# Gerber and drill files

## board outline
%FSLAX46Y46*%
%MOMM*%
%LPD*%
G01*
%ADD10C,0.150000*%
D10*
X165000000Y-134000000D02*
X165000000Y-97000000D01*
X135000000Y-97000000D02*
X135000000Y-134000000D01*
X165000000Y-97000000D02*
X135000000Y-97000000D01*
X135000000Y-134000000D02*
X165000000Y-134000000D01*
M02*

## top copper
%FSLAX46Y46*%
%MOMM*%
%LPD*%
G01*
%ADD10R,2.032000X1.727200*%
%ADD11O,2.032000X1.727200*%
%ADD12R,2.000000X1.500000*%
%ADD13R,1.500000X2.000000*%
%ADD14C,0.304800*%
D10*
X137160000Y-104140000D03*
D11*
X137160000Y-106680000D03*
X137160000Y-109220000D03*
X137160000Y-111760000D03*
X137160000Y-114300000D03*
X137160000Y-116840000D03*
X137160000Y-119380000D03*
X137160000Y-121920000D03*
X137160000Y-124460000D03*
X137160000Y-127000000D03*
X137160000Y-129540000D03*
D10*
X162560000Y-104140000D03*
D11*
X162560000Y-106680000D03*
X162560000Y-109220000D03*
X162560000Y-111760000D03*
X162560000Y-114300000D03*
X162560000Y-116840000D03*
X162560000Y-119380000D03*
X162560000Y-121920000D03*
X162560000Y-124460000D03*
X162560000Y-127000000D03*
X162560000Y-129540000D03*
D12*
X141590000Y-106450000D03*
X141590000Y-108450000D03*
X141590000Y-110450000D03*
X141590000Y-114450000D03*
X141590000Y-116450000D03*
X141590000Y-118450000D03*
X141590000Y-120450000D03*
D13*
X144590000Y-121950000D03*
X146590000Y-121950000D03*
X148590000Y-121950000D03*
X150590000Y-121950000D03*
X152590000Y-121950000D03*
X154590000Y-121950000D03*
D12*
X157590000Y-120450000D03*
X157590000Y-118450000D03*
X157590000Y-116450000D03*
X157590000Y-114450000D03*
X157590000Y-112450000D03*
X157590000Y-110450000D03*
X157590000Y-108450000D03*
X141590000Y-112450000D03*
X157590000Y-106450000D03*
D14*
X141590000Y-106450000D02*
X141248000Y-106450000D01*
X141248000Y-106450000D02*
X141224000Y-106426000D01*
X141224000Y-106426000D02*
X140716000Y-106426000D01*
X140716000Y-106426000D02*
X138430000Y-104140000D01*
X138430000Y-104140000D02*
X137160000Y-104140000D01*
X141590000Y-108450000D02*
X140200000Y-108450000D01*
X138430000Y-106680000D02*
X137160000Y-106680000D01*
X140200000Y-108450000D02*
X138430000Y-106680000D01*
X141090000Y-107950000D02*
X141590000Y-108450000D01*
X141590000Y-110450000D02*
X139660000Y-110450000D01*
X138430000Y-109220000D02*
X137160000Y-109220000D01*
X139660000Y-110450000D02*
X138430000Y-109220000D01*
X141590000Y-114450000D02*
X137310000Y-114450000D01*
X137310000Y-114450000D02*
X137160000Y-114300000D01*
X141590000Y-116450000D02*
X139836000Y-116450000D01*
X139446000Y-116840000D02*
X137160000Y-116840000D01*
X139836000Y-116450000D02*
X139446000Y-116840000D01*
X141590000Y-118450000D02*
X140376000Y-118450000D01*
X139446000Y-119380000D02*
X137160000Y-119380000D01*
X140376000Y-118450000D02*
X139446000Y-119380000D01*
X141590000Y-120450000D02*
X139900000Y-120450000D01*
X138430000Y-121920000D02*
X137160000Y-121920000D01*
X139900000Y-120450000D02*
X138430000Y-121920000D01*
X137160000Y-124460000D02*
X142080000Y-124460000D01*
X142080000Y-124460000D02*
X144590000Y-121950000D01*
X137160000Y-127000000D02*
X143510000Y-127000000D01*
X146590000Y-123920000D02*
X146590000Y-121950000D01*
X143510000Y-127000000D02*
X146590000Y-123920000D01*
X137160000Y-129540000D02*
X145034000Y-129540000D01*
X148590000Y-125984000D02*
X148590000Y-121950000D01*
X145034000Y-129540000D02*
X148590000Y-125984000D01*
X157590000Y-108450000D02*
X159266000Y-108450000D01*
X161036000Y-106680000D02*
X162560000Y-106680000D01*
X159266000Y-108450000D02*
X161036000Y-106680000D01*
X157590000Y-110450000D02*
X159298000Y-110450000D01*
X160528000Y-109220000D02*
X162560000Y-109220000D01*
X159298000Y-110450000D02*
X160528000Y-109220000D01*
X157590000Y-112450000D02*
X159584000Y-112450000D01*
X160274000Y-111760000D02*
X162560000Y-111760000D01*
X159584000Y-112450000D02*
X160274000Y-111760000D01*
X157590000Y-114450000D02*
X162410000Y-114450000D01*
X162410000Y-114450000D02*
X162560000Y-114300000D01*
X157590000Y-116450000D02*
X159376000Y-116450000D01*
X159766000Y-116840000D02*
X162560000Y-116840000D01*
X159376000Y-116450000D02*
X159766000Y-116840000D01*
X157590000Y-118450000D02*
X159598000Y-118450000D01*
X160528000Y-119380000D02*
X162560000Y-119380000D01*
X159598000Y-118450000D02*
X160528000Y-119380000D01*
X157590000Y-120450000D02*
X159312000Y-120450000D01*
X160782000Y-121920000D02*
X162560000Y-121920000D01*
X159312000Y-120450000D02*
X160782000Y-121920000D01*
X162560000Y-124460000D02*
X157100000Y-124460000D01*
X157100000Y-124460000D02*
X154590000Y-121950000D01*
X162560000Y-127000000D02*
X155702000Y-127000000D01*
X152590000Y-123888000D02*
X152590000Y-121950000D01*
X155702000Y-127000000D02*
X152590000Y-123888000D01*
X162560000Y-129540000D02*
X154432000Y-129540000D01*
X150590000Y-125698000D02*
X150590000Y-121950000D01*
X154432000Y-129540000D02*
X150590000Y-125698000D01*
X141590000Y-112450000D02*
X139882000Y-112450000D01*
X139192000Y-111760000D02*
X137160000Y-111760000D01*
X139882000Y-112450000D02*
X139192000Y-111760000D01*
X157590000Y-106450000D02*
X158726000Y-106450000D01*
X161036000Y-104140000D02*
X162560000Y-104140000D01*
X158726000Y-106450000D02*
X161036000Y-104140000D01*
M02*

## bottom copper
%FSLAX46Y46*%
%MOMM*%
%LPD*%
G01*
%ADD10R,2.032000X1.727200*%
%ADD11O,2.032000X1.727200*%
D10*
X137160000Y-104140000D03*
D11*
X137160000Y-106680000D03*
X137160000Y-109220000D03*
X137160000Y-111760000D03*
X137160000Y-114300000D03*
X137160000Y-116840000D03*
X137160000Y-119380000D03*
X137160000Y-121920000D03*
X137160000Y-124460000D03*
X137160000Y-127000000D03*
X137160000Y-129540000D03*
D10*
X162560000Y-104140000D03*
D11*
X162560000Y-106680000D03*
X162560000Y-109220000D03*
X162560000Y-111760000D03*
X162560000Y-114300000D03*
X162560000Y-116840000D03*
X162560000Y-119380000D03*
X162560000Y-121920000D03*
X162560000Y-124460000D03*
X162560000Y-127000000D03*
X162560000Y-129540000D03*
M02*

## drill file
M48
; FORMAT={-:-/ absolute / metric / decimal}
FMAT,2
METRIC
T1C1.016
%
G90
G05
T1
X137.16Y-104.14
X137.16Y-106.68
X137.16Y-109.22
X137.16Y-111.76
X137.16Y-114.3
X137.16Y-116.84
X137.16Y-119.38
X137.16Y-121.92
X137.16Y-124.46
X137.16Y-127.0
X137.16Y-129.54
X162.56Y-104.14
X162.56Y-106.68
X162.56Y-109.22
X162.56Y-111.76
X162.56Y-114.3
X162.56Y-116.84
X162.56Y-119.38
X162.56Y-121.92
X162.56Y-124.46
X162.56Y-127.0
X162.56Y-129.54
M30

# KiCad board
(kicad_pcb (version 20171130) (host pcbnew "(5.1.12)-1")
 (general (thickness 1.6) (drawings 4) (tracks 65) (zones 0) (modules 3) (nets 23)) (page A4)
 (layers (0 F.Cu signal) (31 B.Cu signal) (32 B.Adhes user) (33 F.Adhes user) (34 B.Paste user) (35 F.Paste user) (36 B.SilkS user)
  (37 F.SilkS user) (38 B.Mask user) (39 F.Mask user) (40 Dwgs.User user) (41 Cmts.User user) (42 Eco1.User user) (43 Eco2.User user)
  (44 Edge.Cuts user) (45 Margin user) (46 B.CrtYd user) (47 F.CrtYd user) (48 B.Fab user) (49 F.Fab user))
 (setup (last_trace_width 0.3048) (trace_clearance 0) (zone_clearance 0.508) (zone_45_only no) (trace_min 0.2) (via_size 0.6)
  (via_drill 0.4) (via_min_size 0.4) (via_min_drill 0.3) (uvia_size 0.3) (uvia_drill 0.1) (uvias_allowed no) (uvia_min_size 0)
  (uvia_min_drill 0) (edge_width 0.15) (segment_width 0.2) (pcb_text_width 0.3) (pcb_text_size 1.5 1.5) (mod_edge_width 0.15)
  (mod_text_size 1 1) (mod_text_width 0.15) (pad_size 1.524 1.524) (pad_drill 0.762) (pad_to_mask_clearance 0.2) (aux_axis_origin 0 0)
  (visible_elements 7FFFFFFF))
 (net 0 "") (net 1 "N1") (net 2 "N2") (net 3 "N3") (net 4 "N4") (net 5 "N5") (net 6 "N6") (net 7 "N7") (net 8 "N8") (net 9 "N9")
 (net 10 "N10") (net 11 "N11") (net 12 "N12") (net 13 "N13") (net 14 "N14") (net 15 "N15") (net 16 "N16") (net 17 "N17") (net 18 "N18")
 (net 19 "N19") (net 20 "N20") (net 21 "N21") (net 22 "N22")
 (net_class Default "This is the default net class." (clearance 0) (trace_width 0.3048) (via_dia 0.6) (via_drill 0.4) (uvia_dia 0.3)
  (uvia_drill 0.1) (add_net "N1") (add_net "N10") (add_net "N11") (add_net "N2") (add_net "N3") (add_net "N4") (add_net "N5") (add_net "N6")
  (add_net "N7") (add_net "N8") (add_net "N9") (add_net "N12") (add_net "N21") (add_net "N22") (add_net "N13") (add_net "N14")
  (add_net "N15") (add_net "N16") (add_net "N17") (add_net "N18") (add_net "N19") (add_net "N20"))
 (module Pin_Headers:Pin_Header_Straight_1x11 (layer F.Cu) (at 137.16 104.14)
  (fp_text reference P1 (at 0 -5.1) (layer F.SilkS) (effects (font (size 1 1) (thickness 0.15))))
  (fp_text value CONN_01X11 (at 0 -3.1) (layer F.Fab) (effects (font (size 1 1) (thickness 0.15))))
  (pad 1 thru_hole rect (at 0 0) (size 2.032 1.7272) (drill 1.016) (layers *.Cu *.Mask F.SilkS) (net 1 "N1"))
  (pad 2 thru_hole oval (at 0 2.54) (size 2.032 1.7272) (drill 1.016) (layers *.Cu *.Mask F.SilkS) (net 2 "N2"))
  (pad 3 thru_hole oval (at 0 5.08) (size 2.032 1.7272) (drill 1.016) (layers *.Cu *.Mask F.SilkS) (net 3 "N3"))
  (pad 4 thru_hole oval (at 0 7.62) (size 2.032 1.7272) (drill 1.016) (layers *.Cu *.Mask F.SilkS) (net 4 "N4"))
  (pad 5 thru_hole oval (at 0 10.16) (size 2.032 1.7272) (drill 1.016) (layers *.Cu *.Mask F.SilkS) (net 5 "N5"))
  (pad 6 thru_hole oval (at 0 12.7) (size 2.032 1.7272) (drill 1.016) (layers *.Cu *.Mask F.SilkS) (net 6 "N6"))
  (pad 7 thru_hole oval (at 0 15.24) (size 2.032 1.7272) (drill 1.016) (layers *.Cu *.Mask F.SilkS) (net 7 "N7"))
  (pad 8 thru_hole oval (at 0 17.78) (size 2.032 1.7272) (drill 1.016) (layers *.Cu *.Mask F.SilkS) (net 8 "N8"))
  (pad 9 thru_hole oval (at 0 20.32) (size 2.032 1.7272) (drill 1.016) (layers *.Cu *.Mask F.SilkS) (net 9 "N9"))
  (pad 10 thru_hole oval (at 0 22.86) (size 2.032 1.7272) (drill 1.016) (layers *.Cu *.Mask F.SilkS) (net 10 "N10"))
  (pad 11 thru_hole oval (at 0 25.4) (size 2.032 1.7272) (drill 1.016) (layers *.Cu *.Mask F.SilkS) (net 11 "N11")))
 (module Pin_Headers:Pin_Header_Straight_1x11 (layer F.Cu) (at 162.56 104.14)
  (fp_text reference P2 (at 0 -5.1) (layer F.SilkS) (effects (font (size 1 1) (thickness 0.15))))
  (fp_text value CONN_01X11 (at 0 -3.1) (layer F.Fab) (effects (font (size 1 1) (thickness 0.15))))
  (pad 1 thru_hole rect (at 0 0) (size 2.032 1.7272) (drill 1.016) (layers *.Cu *.Mask F.SilkS) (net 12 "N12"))
  (pad 2 thru_hole oval (at 0 2.54) (size 2.032 1.7272) (drill 1.016) (layers *.Cu *.Mask F.SilkS) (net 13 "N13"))
  (pad 3 thru_hole oval (at 0 5.08) (size 2.032 1.7272) (drill 1.016) (layers *.Cu *.Mask F.SilkS) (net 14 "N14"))
  (pad 4 thru_hole oval (at 0 7.62) (size 2.032 1.7272) (drill 1.016) (layers *.Cu *.Mask F.SilkS) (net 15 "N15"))
  (pad 5 thru_hole oval (at 0 10.16) (size 2.032 1.7272) (drill 1.016) (layers *.Cu *.Mask F.SilkS) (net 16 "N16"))
  (pad 6 thru_hole oval (at 0 12.7) (size 2.032 1.7272) (drill 1.016) (layers *.Cu *.Mask F.SilkS) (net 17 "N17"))
  (pad 7 thru_hole oval (at 0 15.24) (size 2.032 1.7272) (drill 1.016) (layers *.Cu *.Mask F.SilkS) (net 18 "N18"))
  (pad 8 thru_hole oval (at 0 17.78) (size 2.032 1.7272) (drill 1.016) (layers *.Cu *.Mask F.SilkS) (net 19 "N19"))
  (pad 9 thru_hole oval (at 0 20.32) (size 2.032 1.7272) (drill 1.016) (layers *.Cu *.Mask F.SilkS) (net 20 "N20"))
  (pad 10 thru_hole oval (at 0 22.86) (size 2.032 1.7272) (drill 1.016) (layers *.Cu *.Mask F.SilkS) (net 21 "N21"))
  (pad 11 thru_hole oval (at 0 25.4) (size 2.032 1.7272) (drill 1.016) (layers *.Cu *.Mask F.SilkS) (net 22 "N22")))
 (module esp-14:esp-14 (layer F.Cu) (at 148.59 107.95)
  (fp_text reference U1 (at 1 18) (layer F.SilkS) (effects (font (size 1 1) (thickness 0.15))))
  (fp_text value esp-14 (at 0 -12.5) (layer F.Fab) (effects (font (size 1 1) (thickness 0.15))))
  (pad 1 smd rect (at -7 -1.5) (size 2 1.5) (layers F.Cu F.Paste F.Mask) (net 1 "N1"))
  (pad 2 smd rect (at -7 0.5) (size 2 1.5) (layers F.Cu F.Paste F.Mask) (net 2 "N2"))
  (pad 3 smd rect (at -7 2.5) (size 2 1.5) (layers F.Cu F.Paste F.Mask) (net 3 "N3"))
  (pad 5 smd rect (at -7 6.5) (size 2 1.5) (layers F.Cu F.Paste F.Mask) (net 5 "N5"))
  (pad 6 smd rect (at -7 8.5) (size 2 1.5) (layers F.Cu F.Paste F.Mask) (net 6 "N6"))
  (pad 7 smd rect (at -7 10.5) (size 2 1.5) (layers F.Cu F.Paste F.Mask) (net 7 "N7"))
  (pad 8 smd rect (at -7 12.5) (size 2 1.5) (layers F.Cu F.Paste F.Mask) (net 8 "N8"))
  (pad 9 smd rect (at -4 14) (size 1.5 2) (layers F.Cu F.Paste F.Mask) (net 9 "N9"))
  (pad 10 smd rect (at -2 14) (size 1.5 2) (layers F.Cu F.Paste F.Mask) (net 10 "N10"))
  (pad 11 smd rect (at 0 14) (size 1.5 2) (layers F.Cu F.Paste F.Mask) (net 11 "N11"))
  (pad 12 smd rect (at 2 14) (size 1.5 2) (layers F.Cu F.Paste F.Mask) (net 22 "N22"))
  (pad 13 smd rect (at 4 14) (size 1.5 2) (layers F.Cu F.Paste F.Mask) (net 21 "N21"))
  (pad 14 smd rect (at 6 14) (size 1.5 2) (layers F.Cu F.Paste F.Mask) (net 20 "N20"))
  (pad 15 smd rect (at 9 12.5) (size 2 1.5) (layers F.Cu F.Paste F.Mask) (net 19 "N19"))
  (pad 16 smd rect (at 9 10.5) (size 2 1.5) (layers F.Cu F.Paste F.Mask) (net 18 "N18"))
  (pad 17 smd rect (at 9 8.5) (size 2 1.5) (layers F.Cu F.Paste F.Mask) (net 17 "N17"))
  (pad 18 smd rect (at 9 6.5) (size 2 1.5) (layers F.Cu F.Paste F.Mask) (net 16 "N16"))
  (pad 19 smd rect (at 9 4.5) (size 2 1.5) (layers F.Cu F.Paste F.Mask) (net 15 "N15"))
  (pad 20 smd rect (at 9 2.5) (size 2 1.5) (layers F.Cu F.Paste F.Mask) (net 14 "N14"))
  (pad 21 smd rect (at 9 0.5) (size 2 1.5) (layers F.Cu F.Paste F.Mask) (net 13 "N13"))
  (pad 4 smd rect (at -7 4.5) (size 2 1.5) (layers F.Cu F.Paste F.Mask) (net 4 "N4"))
  (pad 22 smd rect (at 9 -1.5) (size 2 1.5) (layers F.Cu F.Paste F.Mask) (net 12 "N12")))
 (gr_line (start 165 134) (end 165 97) (angle 90) (layer Edge.Cuts) (width 0.15))
 (gr_line (start 135 97) (end 135 134) (angle 90) (layer Edge.Cuts) (width 0.15))
 (gr_line (start 165 97) (end 135 97) (angle 90) (layer Edge.Cuts) (width 0.15))
 (gr_line (start 135 134) (end 165 134) (angle 90) (layer Edge.Cuts) (width 0.15))
 (segment (start 141.59 106.45) (end 141.248 106.45) (width 0.3048) (layer F.Cu) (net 1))
 (segment (start 141.248 106.45) (end 141.224 106.426) (width 0.3048) (layer F.Cu) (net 1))
 (segment (start 141.224 106.426) (end 140.716 106.426) (width 0.3048) (layer F.Cu) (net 1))
 (segment (start 140.716 106.426) (end 138.43 104.14) (width 0.3048) (layer F.Cu) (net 1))
 (segment (start 138.43 104.14) (end 137.16 104.14) (width 0.3048) (layer F.Cu) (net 1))
 (segment (start 141.59 108.45) (end 140.2 108.45) (width 0.3048) (layer F.Cu) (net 2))
 (segment (start 138.43 106.68) (end 137.16 106.68) (width 0.3048) (layer F.Cu) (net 2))
 (segment (start 140.2 108.45) (end 138.43 106.68) (width 0.3048) (layer F.Cu) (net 2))
 (segment (start 141.09 107.95) (end 141.59 108.45) (width 0.3048) (layer F.Cu) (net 2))
 (segment (start 141.59 110.45) (end 139.66 110.45) (width 0.3048) (layer F.Cu) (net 3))
 (segment (start 138.43 109.22) (end 137.16 109.22) (width 0.3048) (layer F.Cu) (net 3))
 (segment (start 139.66 110.45) (end 138.43 109.22) (width 0.3048) (layer F.Cu) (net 3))
 (segment (start 141.59 114.45) (end 137.31 114.45) (width 0.3048) (layer F.Cu) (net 5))
 (segment (start 137.31 114.45) (end 137.16 114.3) (width 0.3048) (layer F.Cu) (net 5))
 (segment (start 141.59 116.45) (end 139.836 116.45) (width 0.3048) (layer F.Cu) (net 6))
 (segment (start 139.446 116.84) (end 137.16 116.84) (width 0.3048) (layer F.Cu) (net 6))
 (segment (start 139.836 116.45) (end 139.446 116.84) (width 0.3048) (layer F.Cu) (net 6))
 (segment (start 141.59 118.45) (end 140.376 118.45) (width 0.3048) (layer F.Cu) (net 7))
 (segment (start 139.446 119.38) (end 137.16 119.38) (width 0.3048) (layer F.Cu) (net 7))
 (segment (start 140.376 118.45) (end 139.446 119.38) (width 0.3048) (layer F.Cu) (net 7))
 (segment (start 141.59 120.45) (end 139.9 120.45) (width 0.3048) (layer F.Cu) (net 8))
 (segment (start 138.43 121.92) (end 137.16 121.92) (width 0.3048) (layer F.Cu) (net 8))
 (segment (start 139.9 120.45) (end 138.43 121.92) (width 0.3048) (layer F.Cu) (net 8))
 (segment (start 137.16 124.46) (end 142.08 124.46) (width 0.3048) (layer F.Cu) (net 9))
 (segment (start 142.08 124.46) (end 144.59 121.95) (width 0.3048) (layer F.Cu) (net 9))
 (segment (start 137.16 127) (end 143.51 127) (width 0.3048) (layer F.Cu) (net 10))
 (segment (start 146.59 123.92) (end 146.59 121.95) (width 0.3048) (layer F.Cu) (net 10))
 (segment (start 143.51 127) (end 146.59 123.92) (width 0.3048) (layer F.Cu) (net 10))
 (segment (start 137.16 129.54) (end 145.034 129.54) (width 0.3048) (layer F.Cu) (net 11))
 (segment (start 148.59 125.984) (end 148.59 121.95) (width 0.3048) (layer F.Cu) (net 11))
 (segment (start 145.034 129.54) (end 148.59 125.984) (width 0.3048) (layer F.Cu) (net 11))
 (segment (start 157.59 108.45) (end 159.266 108.45) (width 0.3048) (layer F.Cu) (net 13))
 (segment (start 161.036 106.68) (end 162.56 106.68) (width 0.3048) (layer F.Cu) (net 13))
 (segment (start 159.266 108.45) (end 161.036 106.68) (width 0.3048) (layer F.Cu) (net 13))
 (segment (start 157.59 110.45) (end 159.298 110.45) (width 0.3048) (layer F.Cu) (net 14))
 (segment (start 160.528 109.22) (end 162.56 109.22) (width 0.3048) (layer F.Cu) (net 14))
 (segment (start 159.298 110.45) (end 160.528 109.22) (width 0.3048) (layer F.Cu) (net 14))
 (segment (start 157.59 112.45) (end 159.584 112.45) (width 0.3048) (layer F.Cu) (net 15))
 (segment (start 160.274 111.76) (end 162.56 111.76) (width 0.3048) (layer F.Cu) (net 15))
 (segment (start 159.584 112.45) (end 160.274 111.76) (width 0.3048) (layer F.Cu) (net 15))
 (segment (start 157.59 114.45) (end 162.41 114.45) (width 0.3048) (layer F.Cu) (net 16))
 (segment (start 162.41 114.45) (end 162.56 114.3) (width 0.3048) (layer F.Cu) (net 16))
 (segment (start 157.59 116.45) (end 159.376 116.45) (width 0.3048) (layer F.Cu) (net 17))
 (segment (start 159.766 116.84) (end 162.56 116.84) (width 0.3048) (layer F.Cu) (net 17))
 (segment (start 159.376 116.45) (end 159.766 116.84) (width 0.3048) (layer F.Cu) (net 17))
 (segment (start 157.59 118.45) (end 159.598 118.45) (width 0.3048) (layer F.Cu) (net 18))
 (segment (start 160.528 119.38) (end 162.56 119.38) (width 0.3048) (layer F.Cu) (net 18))
 (segment (start 159.598 118.45) (end 160.528 119.38) (width 0.3048) (layer F.Cu) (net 18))
 (segment (start 157.59 120.45) (end 159.312 120.45) (width 0.3048) (layer F.Cu) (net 19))
 (segment (start 160.782 121.92) (end 162.56 121.92) (width 0.3048) (layer F.Cu) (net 19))
 (segment (start 159.312 120.45) (end 160.782 121.92) (width 0.3048) (layer F.Cu) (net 19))
 (segment (start 162.56 124.46) (end 157.1 124.46) (width 0.3048) (layer F.Cu) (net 20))
 (segment (start 157.1 124.46) (end 154.59 121.95) (width 0.3048) (layer F.Cu) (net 20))
 (segment (start 162.56 127) (end 155.702 127) (width 0.3048) (layer F.Cu) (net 21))
 (segment (start 152.59 123.888) (end 152.59 121.95) (width 0.3048) (layer F.Cu) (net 21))
 (segment (start 155.702 127) (end 152.59 123.888) (width 0.3048) (layer F.Cu) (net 21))
 (segment (start 162.56 129.54) (end 154.432 129.54) (width 0.3048) (layer F.Cu) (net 22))
 (segment (start 150.59 125.698) (end 150.59 121.95) (width 0.3048) (layer F.Cu) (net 22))
 (segment (start 154.432 129.54) (end 150.59 125.698) (width 0.3048) (layer F.Cu) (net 22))
 (segment (start 141.59 112.45) (end 139.882 112.45) (width 0.3048) (layer F.Cu) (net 4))
 (segment (start 139.192 111.76) (end 137.16 111.76) (width 0.3048) (layer F.Cu) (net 4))
 (segment (start 139.882 112.45) (end 139.192 111.76) (width 0.3048) (layer F.Cu) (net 4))
 (segment (start 157.59 106.45) (end 158.726 106.45) (width 0.3048) (layer F.Cu) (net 12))
 (segment (start 161.036 104.14) (end 162.56 104.14) (width 0.3048) (layer F.Cu) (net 12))
 (segment (start 158.726 106.45) (end 161.036 104.14) (width 0.3048) (layer F.Cu) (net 12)))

